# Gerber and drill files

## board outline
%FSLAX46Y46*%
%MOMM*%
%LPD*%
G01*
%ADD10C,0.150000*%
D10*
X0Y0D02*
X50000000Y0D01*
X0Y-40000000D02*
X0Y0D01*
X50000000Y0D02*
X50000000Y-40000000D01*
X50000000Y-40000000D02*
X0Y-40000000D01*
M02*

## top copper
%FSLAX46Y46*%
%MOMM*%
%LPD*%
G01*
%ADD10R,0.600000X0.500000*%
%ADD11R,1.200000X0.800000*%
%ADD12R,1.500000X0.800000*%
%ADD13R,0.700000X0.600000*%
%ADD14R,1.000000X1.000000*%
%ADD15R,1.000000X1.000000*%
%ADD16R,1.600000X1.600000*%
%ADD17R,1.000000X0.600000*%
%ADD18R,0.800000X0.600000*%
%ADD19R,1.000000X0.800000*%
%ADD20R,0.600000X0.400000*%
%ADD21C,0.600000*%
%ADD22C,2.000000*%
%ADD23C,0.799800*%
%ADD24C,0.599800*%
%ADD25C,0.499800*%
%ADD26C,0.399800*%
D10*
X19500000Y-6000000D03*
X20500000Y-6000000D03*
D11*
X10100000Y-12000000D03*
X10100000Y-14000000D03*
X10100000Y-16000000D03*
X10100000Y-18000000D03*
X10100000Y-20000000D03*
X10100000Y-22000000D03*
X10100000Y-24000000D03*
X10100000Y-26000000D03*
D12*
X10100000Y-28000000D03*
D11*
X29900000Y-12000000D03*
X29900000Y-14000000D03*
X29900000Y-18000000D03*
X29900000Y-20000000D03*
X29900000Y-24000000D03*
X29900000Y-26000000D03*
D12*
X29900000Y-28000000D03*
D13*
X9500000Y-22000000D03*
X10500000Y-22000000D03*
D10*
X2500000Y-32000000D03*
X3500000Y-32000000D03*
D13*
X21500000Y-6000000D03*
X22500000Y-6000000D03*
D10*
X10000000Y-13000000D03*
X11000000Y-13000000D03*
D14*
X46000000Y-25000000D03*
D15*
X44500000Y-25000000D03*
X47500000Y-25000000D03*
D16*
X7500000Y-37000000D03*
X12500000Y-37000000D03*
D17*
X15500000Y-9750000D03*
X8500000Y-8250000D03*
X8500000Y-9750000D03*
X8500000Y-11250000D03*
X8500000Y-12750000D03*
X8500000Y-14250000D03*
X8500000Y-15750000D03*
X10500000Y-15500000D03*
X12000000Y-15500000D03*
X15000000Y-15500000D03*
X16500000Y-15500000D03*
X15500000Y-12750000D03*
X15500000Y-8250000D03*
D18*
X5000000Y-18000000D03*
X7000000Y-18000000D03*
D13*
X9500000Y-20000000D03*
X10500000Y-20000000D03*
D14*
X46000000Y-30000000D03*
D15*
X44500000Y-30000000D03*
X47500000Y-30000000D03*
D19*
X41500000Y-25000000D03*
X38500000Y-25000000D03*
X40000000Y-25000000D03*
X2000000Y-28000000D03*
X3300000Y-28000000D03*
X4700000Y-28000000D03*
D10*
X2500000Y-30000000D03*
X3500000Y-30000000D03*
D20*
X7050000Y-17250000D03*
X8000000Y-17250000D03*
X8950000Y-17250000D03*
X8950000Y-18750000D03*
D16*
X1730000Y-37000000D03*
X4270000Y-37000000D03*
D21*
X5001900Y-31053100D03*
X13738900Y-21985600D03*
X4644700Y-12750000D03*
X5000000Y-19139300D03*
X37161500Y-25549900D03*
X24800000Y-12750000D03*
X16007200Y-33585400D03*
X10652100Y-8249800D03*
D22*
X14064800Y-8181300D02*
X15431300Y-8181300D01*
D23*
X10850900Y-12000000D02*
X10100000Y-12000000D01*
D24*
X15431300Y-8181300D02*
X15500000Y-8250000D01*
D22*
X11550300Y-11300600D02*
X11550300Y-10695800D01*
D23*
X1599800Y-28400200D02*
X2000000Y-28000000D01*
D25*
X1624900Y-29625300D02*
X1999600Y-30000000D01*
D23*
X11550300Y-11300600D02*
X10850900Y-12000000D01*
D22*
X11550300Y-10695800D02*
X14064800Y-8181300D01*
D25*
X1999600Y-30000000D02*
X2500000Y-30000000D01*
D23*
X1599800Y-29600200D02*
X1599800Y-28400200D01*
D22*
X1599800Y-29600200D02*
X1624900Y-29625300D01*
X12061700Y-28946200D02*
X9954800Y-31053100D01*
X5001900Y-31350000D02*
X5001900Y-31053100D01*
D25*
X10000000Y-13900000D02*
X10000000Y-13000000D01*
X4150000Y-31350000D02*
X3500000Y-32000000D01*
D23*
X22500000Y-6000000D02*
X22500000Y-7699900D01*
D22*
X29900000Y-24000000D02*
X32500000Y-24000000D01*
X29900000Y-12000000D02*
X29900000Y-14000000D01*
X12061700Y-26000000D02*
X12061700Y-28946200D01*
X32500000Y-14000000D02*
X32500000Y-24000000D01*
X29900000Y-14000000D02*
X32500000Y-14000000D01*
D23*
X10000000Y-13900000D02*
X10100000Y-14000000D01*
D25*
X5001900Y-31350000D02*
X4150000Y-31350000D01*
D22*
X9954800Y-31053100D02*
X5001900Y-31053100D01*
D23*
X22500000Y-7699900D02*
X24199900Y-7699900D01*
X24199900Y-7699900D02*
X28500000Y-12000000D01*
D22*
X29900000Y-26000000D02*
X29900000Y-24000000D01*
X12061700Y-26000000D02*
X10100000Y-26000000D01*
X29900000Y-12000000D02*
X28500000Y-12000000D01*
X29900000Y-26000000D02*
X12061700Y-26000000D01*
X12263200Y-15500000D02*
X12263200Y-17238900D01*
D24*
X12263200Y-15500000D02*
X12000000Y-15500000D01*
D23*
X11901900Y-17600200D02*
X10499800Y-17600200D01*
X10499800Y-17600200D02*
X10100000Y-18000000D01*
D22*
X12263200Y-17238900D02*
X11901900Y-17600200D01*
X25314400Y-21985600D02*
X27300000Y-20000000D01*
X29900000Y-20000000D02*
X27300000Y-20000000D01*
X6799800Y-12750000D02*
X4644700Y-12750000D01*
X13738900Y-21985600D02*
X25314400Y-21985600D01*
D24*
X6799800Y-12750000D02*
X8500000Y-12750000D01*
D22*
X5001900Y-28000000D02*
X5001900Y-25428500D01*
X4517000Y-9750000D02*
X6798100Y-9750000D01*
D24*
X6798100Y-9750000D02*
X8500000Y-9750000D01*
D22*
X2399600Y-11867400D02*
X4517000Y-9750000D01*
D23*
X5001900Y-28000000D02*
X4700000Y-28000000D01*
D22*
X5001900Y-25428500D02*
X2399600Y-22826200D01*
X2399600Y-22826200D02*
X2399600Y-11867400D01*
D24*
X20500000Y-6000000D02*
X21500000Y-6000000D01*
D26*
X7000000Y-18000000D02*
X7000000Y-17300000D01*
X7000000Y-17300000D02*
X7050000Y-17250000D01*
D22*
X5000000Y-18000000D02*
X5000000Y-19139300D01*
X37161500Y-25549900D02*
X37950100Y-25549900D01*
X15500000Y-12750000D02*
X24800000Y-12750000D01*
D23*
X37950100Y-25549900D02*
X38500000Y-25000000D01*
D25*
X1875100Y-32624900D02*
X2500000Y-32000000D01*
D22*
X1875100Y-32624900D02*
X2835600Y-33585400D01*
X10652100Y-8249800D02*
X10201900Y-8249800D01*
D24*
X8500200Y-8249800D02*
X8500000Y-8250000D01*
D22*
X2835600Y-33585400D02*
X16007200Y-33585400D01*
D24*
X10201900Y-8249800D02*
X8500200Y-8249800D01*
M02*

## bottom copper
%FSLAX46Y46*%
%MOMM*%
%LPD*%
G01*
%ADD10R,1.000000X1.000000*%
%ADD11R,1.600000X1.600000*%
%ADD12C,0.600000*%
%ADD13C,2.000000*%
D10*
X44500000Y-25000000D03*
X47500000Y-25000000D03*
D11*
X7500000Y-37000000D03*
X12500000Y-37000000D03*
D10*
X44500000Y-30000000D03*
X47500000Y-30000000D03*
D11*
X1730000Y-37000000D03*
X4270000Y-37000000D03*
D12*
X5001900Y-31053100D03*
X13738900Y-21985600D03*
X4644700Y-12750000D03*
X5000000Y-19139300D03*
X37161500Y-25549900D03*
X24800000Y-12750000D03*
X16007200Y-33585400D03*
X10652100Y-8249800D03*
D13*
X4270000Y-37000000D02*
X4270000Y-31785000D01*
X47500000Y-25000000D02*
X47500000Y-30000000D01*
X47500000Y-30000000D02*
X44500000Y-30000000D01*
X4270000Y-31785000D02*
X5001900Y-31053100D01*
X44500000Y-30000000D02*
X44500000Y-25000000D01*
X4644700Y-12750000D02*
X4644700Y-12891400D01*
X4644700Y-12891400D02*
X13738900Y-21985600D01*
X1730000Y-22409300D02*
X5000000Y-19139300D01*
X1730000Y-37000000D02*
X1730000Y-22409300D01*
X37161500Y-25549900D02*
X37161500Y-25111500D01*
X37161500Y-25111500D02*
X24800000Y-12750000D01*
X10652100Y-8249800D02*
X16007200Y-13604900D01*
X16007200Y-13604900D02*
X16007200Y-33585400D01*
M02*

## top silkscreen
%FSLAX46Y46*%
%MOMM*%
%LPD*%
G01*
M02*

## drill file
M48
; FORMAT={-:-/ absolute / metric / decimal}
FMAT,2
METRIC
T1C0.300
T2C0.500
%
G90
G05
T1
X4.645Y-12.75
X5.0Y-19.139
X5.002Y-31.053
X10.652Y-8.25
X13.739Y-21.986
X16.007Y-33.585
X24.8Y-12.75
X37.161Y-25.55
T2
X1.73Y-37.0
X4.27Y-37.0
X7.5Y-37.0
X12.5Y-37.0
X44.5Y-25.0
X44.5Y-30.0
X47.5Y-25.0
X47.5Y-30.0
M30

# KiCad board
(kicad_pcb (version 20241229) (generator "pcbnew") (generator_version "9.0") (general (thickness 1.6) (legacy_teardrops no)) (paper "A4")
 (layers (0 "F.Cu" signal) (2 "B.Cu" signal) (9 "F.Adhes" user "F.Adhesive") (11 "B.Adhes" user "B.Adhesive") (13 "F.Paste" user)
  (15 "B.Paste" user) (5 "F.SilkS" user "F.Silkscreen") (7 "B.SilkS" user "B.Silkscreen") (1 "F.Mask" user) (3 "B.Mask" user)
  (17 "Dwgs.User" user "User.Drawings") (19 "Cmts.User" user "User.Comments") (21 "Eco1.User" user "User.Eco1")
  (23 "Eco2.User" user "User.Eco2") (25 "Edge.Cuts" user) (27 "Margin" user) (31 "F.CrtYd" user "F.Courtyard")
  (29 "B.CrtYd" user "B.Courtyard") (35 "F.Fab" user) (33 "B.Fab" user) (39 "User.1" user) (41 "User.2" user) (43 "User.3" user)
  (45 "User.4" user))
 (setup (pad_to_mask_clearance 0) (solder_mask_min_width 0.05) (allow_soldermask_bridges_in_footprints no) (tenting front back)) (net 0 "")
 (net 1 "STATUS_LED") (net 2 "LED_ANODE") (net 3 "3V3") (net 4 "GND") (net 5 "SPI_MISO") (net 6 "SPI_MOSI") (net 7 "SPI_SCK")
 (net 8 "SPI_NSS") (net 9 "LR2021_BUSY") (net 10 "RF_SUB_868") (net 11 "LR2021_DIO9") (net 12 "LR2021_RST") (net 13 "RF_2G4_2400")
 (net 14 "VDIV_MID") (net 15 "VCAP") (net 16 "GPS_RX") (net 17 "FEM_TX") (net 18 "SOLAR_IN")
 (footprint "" (layer "F.Cu") (at 20 6)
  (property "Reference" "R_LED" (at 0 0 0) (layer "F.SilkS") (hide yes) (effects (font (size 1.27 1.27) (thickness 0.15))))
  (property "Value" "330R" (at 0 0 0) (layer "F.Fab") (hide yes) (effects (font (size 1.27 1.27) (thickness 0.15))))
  (pad "1" smd rect (at -0.5 0) (size 0.6 0.5) (layers "F.Cu" "F.Mask") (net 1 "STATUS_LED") (thermal_bridge_angle 45))
  (pad "2" smd rect (at 0.5 0) (size 0.6 0.5) (layers "F.Cu" "F.Mask") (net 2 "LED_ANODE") (thermal_bridge_angle 45)))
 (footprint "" (layer "F.Cu") (at 20 20)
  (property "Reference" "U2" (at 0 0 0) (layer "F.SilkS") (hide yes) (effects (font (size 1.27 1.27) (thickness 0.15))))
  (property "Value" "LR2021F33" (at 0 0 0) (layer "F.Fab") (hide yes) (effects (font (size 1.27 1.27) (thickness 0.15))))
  (pad "1" smd rect (at -9.9 -8) (size 1.2 0.8) (layers "F.Cu" "F.Mask") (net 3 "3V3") (thermal_bridge_angle 45))
  (pad "2" smd rect (at -9.9 -6) (size 1.2 0.8) (layers "F.Cu" "F.Mask") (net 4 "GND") (thermal_bridge_angle 45))
  (pad "3" smd rect (at -9.9 -4) (size 1.2 0.8) (layers "F.Cu" "F.Mask") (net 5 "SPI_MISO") (thermal_bridge_angle 45))
  (pad "4" smd rect (at -9.9 -2) (size 1.2 0.8) (layers "F.Cu" "F.Mask") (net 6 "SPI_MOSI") (thermal_bridge_angle 45))
  (pad "5" smd rect (at -9.9 0) (size 1.2 0.8) (layers "F.Cu" "F.Mask") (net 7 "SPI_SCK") (thermal_bridge_angle 45))
  (pad "6" smd rect (at -9.9 2) (size 1.2 0.8) (layers "F.Cu" "F.Mask") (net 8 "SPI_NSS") (thermal_bridge_angle 45))
  (pad "7" smd rect (at -9.9 4) (size 1.2 0.8) (layers "F.Cu" "F.Mask") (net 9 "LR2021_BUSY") (thermal_bridge_angle 45))
  (pad "8" smd rect (at -9.9 6) (size 1.2 0.8) (layers "F.Cu" "F.Mask") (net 4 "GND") (thermal_bridge_angle 45))
  (pad "9" smd rect (at -9.9 8) (size 1.5 0.8) (layers "F.Cu" "F.Mask") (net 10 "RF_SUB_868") (thermal_bridge_angle 45))
  (pad "10" smd rect (at 9.9 -8) (size 1.2 0.8) (layers "F.Cu" "F.Mask") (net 4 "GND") (thermal_bridge_angle 45))
  (pad "11" smd rect (at 9.9 -6) (size 1.2 0.8) (layers "F.Cu" "F.Mask") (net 4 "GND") (thermal_bridge_angle 45))
  (pad "13" smd rect (at 9.9 -2) (size 1.2 0.8) (layers "F.Cu" "F.Mask") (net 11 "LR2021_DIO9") (thermal_bridge_angle 45))
  (pad "14" smd rect (at 9.9 0) (size 1.2 0.8) (layers "F.Cu" "F.Mask") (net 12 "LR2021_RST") (thermal_bridge_angle 45))
  (pad "16" smd rect (at 9.9 4) (size 1.2 0.8) (layers "F.Cu" "F.Mask") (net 4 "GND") (thermal_bridge_angle 45))
  (pad "17" smd rect (at 9.9 6) (size 1.2 0.8) (layers "F.Cu" "F.Mask") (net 4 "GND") (thermal_bridge_angle 45))
  (pad "18" smd rect (at 9.9 8) (size 1.5 0.8) (layers "F.Cu" "F.Mask") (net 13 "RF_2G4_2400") (thermal_bridge_angle 45)))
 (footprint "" (layer "F.Cu") (at 10 22)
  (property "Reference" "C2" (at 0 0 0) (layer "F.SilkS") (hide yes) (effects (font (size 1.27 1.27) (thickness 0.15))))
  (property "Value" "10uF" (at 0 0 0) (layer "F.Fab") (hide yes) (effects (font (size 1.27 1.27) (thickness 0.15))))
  (pad "1" smd rect (at -0.5 0) (size 0.7 0.6) (layers "F.Cu" "F.Mask") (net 3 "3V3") (thermal_bridge_angle 45))
  (pad "2" smd rect (at 0.5 0) (size 0.7 0.6) (layers "F.Cu" "F.Mask") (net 4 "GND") (thermal_bridge_angle 45)))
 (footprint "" (layer "F.Cu") (at 3 32)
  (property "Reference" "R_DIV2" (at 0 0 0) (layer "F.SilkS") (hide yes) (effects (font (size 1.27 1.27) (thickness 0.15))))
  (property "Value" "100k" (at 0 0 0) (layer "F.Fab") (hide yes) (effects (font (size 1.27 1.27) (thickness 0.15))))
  (pad "1" smd rect (at -0.5 0) (size 0.6 0.5) (layers "F.Cu" "F.Mask") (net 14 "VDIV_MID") (thermal_bridge_angle 45))
  (pad "2" smd rect (at 0.5 0) (size 0.6 0.5) (layers "F.Cu" "F.Mask") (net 4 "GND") (thermal_bridge_angle 45)))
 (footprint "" (layer "F.Cu") (at 22 6)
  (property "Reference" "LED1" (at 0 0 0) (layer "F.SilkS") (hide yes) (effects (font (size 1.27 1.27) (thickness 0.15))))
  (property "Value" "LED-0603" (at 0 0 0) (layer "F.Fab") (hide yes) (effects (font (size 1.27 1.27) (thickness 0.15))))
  (pad "A" smd rect (at -0.5 0) (size 0.7 0.6) (layers "F.Cu" "F.Mask") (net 2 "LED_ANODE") (thermal_bridge_angle 45))
  (pad "K" smd rect (at 0.5 0) (size 0.7 0.6) (layers "F.Cu" "F.Mask") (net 4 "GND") (thermal_bridge_angle 45)))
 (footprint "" (layer "F.Cu") (at 10.5 13)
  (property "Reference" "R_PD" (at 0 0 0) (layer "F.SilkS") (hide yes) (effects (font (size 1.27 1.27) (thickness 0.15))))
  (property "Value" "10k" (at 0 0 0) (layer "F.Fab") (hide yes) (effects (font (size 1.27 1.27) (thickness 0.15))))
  (pad "1" smd rect (at -0.5 0) (size 0.6 0.5) (layers "F.Cu" "F.Mask") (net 4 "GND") (thermal_bridge_angle 45))
  (pad "2" smd rect (at 0.5 0) (size 0.6 0.5) (layers "F.Cu" "F.Mask") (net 5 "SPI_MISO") (thermal_bridge_angle 45)))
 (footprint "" (layer "F.Cu") (at 46 25)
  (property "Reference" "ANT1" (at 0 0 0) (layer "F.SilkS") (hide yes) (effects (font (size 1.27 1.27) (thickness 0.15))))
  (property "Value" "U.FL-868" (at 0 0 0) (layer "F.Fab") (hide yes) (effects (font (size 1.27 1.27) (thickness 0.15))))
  (pad "1" smd rect (at 0 0) (size 1 1) (layers "F.Cu" "F.Mask") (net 10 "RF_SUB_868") (thermal_bridge_angle 45))
  (pad "2" thru_hole rect (at -1.5 0) (size 1 1) (drill 0.5) (layers "*.Cu" "*.Mask") (remove_unused_layers no) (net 4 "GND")
   (thermal_bridge_angle 45))
  (pad "3" thru_hole rect (at 1.5 0) (size 1 1) (drill 0.5) (layers "*.Cu" "*.Mask") (remove_unused_layers no) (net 4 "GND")
   (thermal_bridge_angle 45)))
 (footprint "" (layer "F.Cu") (at 10 37)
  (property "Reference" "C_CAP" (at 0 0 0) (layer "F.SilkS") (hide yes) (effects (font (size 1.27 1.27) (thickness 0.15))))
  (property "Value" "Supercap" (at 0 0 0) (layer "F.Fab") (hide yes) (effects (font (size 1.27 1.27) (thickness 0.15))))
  (pad "1" thru_hole rect (at -2.5 0) (size 1.6 1.6) (drill 0.5) (layers "*.Cu" "*.Mask") (remove_unused_layers no) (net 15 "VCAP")
   (thermal_bridge_angle 45))
  (pad "2" thru_hole rect (at 2.5 0) (size 1.6 1.6) (drill 0.5) (layers "*.Cu" "*.Mask") (remove_unused_layers no) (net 4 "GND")
   (thermal_bridge_angle 45)))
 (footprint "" (layer "F.Cu") (at 12 12)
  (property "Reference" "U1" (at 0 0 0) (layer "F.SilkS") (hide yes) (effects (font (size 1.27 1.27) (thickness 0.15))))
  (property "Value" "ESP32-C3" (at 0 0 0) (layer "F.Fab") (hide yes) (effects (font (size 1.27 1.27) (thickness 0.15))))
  (pad "GND" smd rect (at 3.5 -2.25) (size 1 0.6) (layers "F.Cu" "F.Mask") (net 4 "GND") (thermal_bridge_angle 45))
  (pad "GPIO0" smd rect (at -3.5 -3.75) (size 1 0.6) (layers "F.Cu" "F.Mask") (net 14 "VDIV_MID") (thermal_bridge_angle 45))
  (pad "GPIO1" smd rect (at -3.5 -2.25) (size 1 0.6) (layers "F.Cu" "F.Mask") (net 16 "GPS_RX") (thermal_bridge_angle 45))
  (pad "GPIO2" smd rect (at -3.5 -0.75) (size 1 0.6) (layers "F.Cu" "F.Mask") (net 5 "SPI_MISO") (thermal_bridge_angle 45))
  (pad "GPIO3" smd rect (at -3.5 0.75) (size 1 0.6) (layers "F.Cu" "F.Mask") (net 12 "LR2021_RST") (thermal_bridge_angle 45))
  (pad "GPIO4" smd rect (at -3.5 2.25) (size 1 0.6) (layers "F.Cu" "F.Mask") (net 9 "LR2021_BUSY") (thermal_bridge_angle 45))
  (pad "GPIO5" smd rect (at -3.5 3.75) (size 1 0.6) (layers "F.Cu" "F.Mask") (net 11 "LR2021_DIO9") (thermal_bridge_angle 45))
  (pad "GPIO6" smd rect (at -1.5 3.5) (size 1 0.6) (layers "F.Cu" "F.Mask") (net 7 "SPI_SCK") (thermal_bridge_angle 45))
  (pad "GPIO7" smd rect (at 0 3.5) (size 1 0.6) (layers "F.Cu" "F.Mask") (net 6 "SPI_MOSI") (thermal_bridge_angle 45))
  (pad "GPIO9" smd rect (at 3 3.5) (size 1 0.6) (layers "F.Cu" "F.Mask") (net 1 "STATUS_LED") (thermal_bridge_angle 45))
  (pad "GPIO10" smd rect (at 4.5 3.5) (size 1 0.6) (layers "F.Cu" "F.Mask") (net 8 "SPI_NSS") (thermal_bridge_angle 45))
  (pad "GPIO19" smd rect (at 3.5 0.75) (size 1 0.6) (layers "F.Cu" "F.Mask") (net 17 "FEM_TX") (thermal_bridge_angle 45))
  (pad "VCC" smd rect (at 3.5 -3.75) (size 1 0.6) (layers "F.Cu" "F.Mask") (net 3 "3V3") (thermal_bridge_angle 45)))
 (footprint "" (layer "F.Cu") (at 6 18)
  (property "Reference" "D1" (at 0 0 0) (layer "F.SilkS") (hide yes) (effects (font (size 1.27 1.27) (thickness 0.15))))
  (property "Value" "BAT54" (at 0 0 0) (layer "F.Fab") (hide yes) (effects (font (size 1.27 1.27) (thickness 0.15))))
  (pad "A" smd rect (at -1 0) (size 0.8 0.6) (layers "F.Cu" "F.Mask") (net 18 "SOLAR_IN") (thermal_bridge_angle 45))
  (pad "K" smd rect (at 1 0) (size 0.8 0.6) (layers "F.Cu" "F.Mask") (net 15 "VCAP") (thermal_bridge_angle 45)))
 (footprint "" (layer "F.Cu") (at 10 20)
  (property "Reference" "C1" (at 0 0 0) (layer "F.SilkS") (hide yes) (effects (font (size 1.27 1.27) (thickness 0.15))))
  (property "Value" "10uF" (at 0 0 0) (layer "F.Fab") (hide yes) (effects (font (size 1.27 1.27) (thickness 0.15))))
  (pad "1" smd rect (at -0.5 0) (size 0.7 0.6) (layers "F.Cu" "F.Mask") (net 15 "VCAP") (thermal_bridge_angle 45))
  (pad "2" smd rect (at 0.5 0) (size 0.7 0.6) (layers "F.Cu" "F.Mask") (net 4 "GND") (thermal_bridge_angle 45)))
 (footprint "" (layer "F.Cu") (at 46 30)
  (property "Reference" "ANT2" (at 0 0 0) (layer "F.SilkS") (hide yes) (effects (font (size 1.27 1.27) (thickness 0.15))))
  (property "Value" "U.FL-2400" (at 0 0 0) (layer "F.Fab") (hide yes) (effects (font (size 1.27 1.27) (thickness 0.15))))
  (pad "1" smd rect (at 0 0) (size 1 1) (layers "F.Cu" "F.Mask") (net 13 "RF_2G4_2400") (thermal_bridge_angle 45))
  (pad "2" thru_hole rect (at -1.5 0) (size 1 1) (drill 0.5) (layers "*.Cu" "*.Mask") (remove_unused_layers no) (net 4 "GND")
   (thermal_bridge_angle 45))
  (pad "3" thru_hole rect (at 1.5 0) (size 1 1) (drill 0.5) (layers "*.Cu" "*.Mask") (remove_unused_layers no) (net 4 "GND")
   (thermal_bridge_angle 45)))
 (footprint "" (layer "F.Cu") (at 40 25)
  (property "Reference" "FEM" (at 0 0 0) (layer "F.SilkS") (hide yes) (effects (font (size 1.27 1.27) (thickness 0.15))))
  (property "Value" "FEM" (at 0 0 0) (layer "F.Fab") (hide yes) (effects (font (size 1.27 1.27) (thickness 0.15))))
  (pad "GND" smd rect (at 1.5 0) (size 1 0.8) (layers "F.Cu" "F.Mask") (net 4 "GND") (thermal_bridge_angle 45))
  (pad "TX" smd rect (at -1.5 0) (size 1 0.8) (layers "F.Cu" "F.Mask") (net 17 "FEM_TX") (thermal_bridge_angle 45))
  (pad "VCC" smd rect (at 0 0) (size 1 0.8) (layers "F.Cu" "F.Mask") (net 3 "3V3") (thermal_bridge_angle 45)))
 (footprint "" (layer "F.Cu") (at 4 28)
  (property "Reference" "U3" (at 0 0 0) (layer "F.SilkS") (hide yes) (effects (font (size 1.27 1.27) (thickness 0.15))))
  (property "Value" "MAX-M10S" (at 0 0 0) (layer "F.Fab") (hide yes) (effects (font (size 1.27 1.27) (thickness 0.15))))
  (pad "1" smd rect (at -2 0) (size 1 0.8) (layers "F.Cu" "F.Mask") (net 3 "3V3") (thermal_bridge_angle 45))
  (pad "2" smd rect (at -0.7 0) (size 1 0.8) (layers "F.Cu" "F.Mask") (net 4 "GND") (thermal_bridge_angle 45))
  (pad "3" smd rect (at 0.7 0) (size 1 0.8) (layers "F.Cu" "F.Mask") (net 16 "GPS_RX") (thermal_bridge_angle 45)))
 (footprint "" (layer "F.Cu") (at 3 30)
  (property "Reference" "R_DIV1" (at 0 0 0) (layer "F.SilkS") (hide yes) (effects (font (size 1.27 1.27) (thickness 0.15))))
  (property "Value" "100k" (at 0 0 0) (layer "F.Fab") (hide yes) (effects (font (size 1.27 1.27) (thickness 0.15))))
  (pad "1" smd rect (at -0.5 0) (size 0.6 0.5) (layers "F.Cu" "F.Mask") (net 3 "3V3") (thermal_bridge_angle 45))
  (pad "2" smd rect (at 0.5 0) (size 0.6 0.5) (layers "F.Cu" "F.Mask") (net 14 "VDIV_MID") (thermal_bridge_angle 45)))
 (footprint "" (layer "F.Cu") (at 8 18)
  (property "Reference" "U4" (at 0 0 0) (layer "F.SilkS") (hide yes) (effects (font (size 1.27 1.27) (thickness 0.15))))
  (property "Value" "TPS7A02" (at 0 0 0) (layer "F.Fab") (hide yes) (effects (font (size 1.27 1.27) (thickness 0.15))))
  (pad "1" smd rect (at -0.95 -0.75) (size 0.6 0.4) (layers "F.Cu" "F.Mask") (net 15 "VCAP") (thermal_bridge_angle 45))
  (pad "2" smd rect (at 0 -0.75) (size 0.6 0.4) (layers "F.Cu" "F.Mask") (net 4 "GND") (thermal_bridge_angle 45))
  (pad "3" smd rect (at 0.95 -0.75) (size 0.6 0.4) (layers "F.Cu" "F.Mask") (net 15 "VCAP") (thermal_bridge_angle 45))
  (pad "4" smd rect (at 0.95 0.75) (size 0.6 0.4) (layers "F.Cu" "F.Mask") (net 3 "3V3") (thermal_bridge_angle 45)))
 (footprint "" (layer "F.Cu") (at 3 37)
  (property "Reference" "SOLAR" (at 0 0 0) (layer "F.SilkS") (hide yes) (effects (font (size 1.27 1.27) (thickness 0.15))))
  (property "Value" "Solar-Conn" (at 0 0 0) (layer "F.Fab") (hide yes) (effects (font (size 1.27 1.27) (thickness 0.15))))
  (pad "1" thru_hole rect (at -1.27 0) (size 1.6 1.6) (drill 0.5) (layers "*.Cu" "*.Mask") (remove_unused_layers no) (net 18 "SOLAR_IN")
   (thermal_bridge_angle 45))
  (pad "2" thru_hole rect (at 1.27 0) (size 1.6 1.6) (drill 0.5) (layers "*.Cu" "*.Mask") (remove_unused_layers no) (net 4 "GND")
   (thermal_bridge_angle 45)))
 (gr_line (start 0 0) (end 50 0) (stroke (width 0.15) (type default)) (layer "Edge.Cuts"))
 (gr_line (start 0 40) (end 0 0) (stroke (width 0.15) (type default)) (layer "Edge.Cuts"))
 (gr_line (start 50 0) (end 50 40) (stroke (width 0.15) (type default)) (layer "Edge.Cuts"))
 (gr_line (start 50 40) (end 0 40) (stroke (width 0.15) (type default)) (layer "Edge.Cuts"))
 (segment (start 14.0648 8.1813) (end 15.4313 8.1813) (width 2) (layer "F.Cu") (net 3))
 (segment (start 10.8509 12) (end 10.1 12) (width 0.7998) (layer "F.Cu") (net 3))
 (segment (start 15.4313 8.1813) (end 15.5 8.25) (width 0.5998) (layer "F.Cu") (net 3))
 (segment (start 11.5503 11.3006) (end 11.5503 10.6958) (width 2) (layer "F.Cu") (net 3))
 (segment (start 1.5998 28.4002) (end 2 28) (width 0.7998) (layer "F.Cu") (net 3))
 (segment (start 1.6249 29.6253) (end 1.9996 30) (width 0.4998) (layer "F.Cu") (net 3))
 (segment (start 11.5503 11.3006) (end 10.8509 12) (width 0.7998) (layer "F.Cu") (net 3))
 (segment (start 11.5503 10.6958) (end 14.0648 8.1813) (width 2) (layer "F.Cu") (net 3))
 (segment (start 1.9996 30) (end 2.5 30) (width 0.4998) (layer "F.Cu") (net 3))
 (segment (start 1.5998 29.6002) (end 1.5998 28.4002) (width 0.7998) (layer "F.Cu") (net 3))
 (segment (start 1.5998 29.6002) (end 1.6249 29.6253) (width 2) (layer "F.Cu") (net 3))
 (segment (start 12.0617 28.9462) (end 9.9548 31.0531) (width 2) (layer "F.Cu") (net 4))
 (segment (start 5.0019 31.35) (end 5.0019 31.0531) (width 2) (layer "F.Cu") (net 4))
 (segment (start 10 13.9) (end 10 13) (width 0.4998) (layer "F.Cu") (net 4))
 (segment (start 4.15 31.35) (end 3.5 32) (width 0.4998) (layer "F.Cu") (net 4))
 (segment (start 22.5 6) (end 22.5 7.6999) (width 0.7998) (layer "F.Cu") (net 4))
 (segment (start 29.9 24) (end 32.5 24) (width 2) (layer "F.Cu") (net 4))
 (segment (start 29.9 12) (end 29.9 14) (width 2) (layer "F.Cu") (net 4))
 (segment (start 12.0617 26) (end 12.0617 28.9462) (width 2) (layer "F.Cu") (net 4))
 (segment (start 32.5 14) (end 32.5 24) (width 2) (layer "F.Cu") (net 4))
 (segment (start 29.9 14) (end 32.5 14) (width 2) (layer "F.Cu") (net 4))
 (segment (start 10 13.9) (end 10.1 14) (width 0.7998) (layer "F.Cu") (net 4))
 (segment (start 5.0019 31.35) (end 4.15 31.35) (width 0.4998) (layer "F.Cu") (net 4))
 (segment (start 9.9548 31.0531) (end 5.0019 31.0531) (width 2) (layer "F.Cu") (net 4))
 (segment (start 22.5 7.6999) (end 24.1999 7.6999) (width 0.7998) (layer "F.Cu") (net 4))
 (segment (start 24.1999 7.6999) (end 28.5 12) (width 0.7998) (layer "F.Cu") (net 4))
 (segment (start 29.9 26) (end 29.9 24) (width 2) (layer "F.Cu") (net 4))
 (segment (start 12.0617 26) (end 10.1 26) (width 2) (layer "F.Cu") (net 4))
 (segment (start 29.9 12) (end 28.5 12) (width 2) (layer "F.Cu") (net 4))
 (segment (start 29.9 26) (end 12.0617 26) (width 2) (layer "F.Cu") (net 4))
 (via (at 5.0019 31.0531) (size 0.6) (drill 0.3) (layers "F.Cu" "B.Cu") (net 4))
 (segment (start 4.27 37) (end 4.27 31.785) (width 2) (layer "B.Cu") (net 4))
 (segment (start 47.5 25) (end 47.5 30) (width 2) (layer "B.Cu") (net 4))
 (segment (start 47.5 30) (end 44.5 30) (width 2) (layer "B.Cu") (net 4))
 (segment (start 4.27 31.785) (end 5.0019 31.0531) (width 2) (layer "B.Cu") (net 4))
 (segment (start 44.5 30) (end 44.5 25) (width 2) (layer "B.Cu") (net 4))
 (segment (start 12.2632 15.5) (end 12.2632 17.2389) (width 2) (layer "F.Cu") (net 6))
 (segment (start 12.2632 15.5) (end 12 15.5) (width 0.5998) (layer "F.Cu") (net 6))
 (segment (start 11.9019 17.6002) (end 10.4998 17.6002) (width 0.7998) (layer "F.Cu") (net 6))
 (segment (start 10.4998 17.6002) (end 10.1 18) (width 0.7998) (layer "F.Cu") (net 6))
 (segment (start 12.2632 17.2389) (end 11.9019 17.6002) (width 2) (layer "F.Cu") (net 6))
 (segment (start 25.3144 21.9856) (end 27.3 20) (width 2) (layer "F.Cu") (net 12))
 (segment (start 29.9 20) (end 27.3 20) (width 2) (layer "F.Cu") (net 12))
 (segment (start 6.7998 12.75) (end 4.6447 12.75) (width 2) (layer "F.Cu") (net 12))
 (segment (start 13.7389 21.9856) (end 25.3144 21.9856) (width 2) (layer "F.Cu") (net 12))
 (segment (start 6.7998 12.75) (end 8.5 12.75) (width 0.5998) (layer "F.Cu") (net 12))
 (via (at 13.7389 21.9856) (size 0.6) (drill 0.3) (layers "F.Cu" "B.Cu") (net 12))
 (via (at 4.6447 12.75) (size 0.6) (drill 0.3) (layers "F.Cu" "B.Cu") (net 12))
 (segment (start 4.6447 12.75) (end 4.6447 12.8914) (width 2) (layer "B.Cu") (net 12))
 (segment (start 4.6447 12.8914) (end 13.7389 21.9856) (width 2) (layer "B.Cu") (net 12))
 (segment (start 5.0019 28) (end 5.0019 25.4285) (width 2) (layer "F.Cu") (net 16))
 (segment (start 4.517 9.75) (end 6.7981 9.75) (width 2) (layer "F.Cu") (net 16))
 (segment (start 6.7981 9.75) (end 8.5 9.75) (width 0.5998) (layer "F.Cu") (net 16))
 (segment (start 2.3996 11.8674) (end 4.517 9.75) (width 2) (layer "F.Cu") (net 16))
 (segment (start 5.0019 28) (end 4.7 28) (width 0.7998) (layer "F.Cu") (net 16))
 (segment (start 5.0019 25.4285) (end 2.3996 22.8262) (width 2) (layer "F.Cu") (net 16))
 (segment (start 2.3996 22.8262) (end 2.3996 11.8674) (width 2) (layer "F.Cu") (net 16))
 (segment (start 20.5 6) (end 21.5 6) (width 0.5998) (layer "F.Cu") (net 2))
 (segment (start 7 18) (end 7 17.3) (width 0.3998) (layer "F.Cu") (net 15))
 (segment (start 7 17.3) (end 7.05 17.25) (width 0.3998) (layer "F.Cu") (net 15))
 (segment (start 5 18) (end 5 19.1393) (width 2) (layer "F.Cu") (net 18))
 (via (at 5 19.1393) (size 0.6) (drill 0.3) (layers "F.Cu" "B.Cu") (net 18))
 (segment (start 1.73 22.4093) (end 5 19.1393) (width 2) (layer "B.Cu") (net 18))
 (segment (start 1.73 37) (end 1.73 22.4093) (width 2) (layer "B.Cu") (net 18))
 (segment (start 37.1615 25.5499) (end 37.9501 25.5499) (width 2) (layer "F.Cu") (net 17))
 (segment (start 15.5 12.75) (end 24.8 12.75) (width 2) (layer "F.Cu") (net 17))
 (segment (start 37.9501 25.5499) (end 38.5 25) (width 0.7998) (layer "F.Cu") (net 17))
 (via (at 37.1615 25.5499) (size 0.6) (drill 0.3) (layers "F.Cu" "B.Cu") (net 17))
 (via (at 24.8 12.75) (size 0.6) (drill 0.3) (layers "F.Cu" "B.Cu") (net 17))
 (segment (start 37.1615 25.5499) (end 37.1615 25.1115) (width 2) (layer "B.Cu") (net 17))
 (segment (start 37.1615 25.1115) (end 24.8 12.75) (width 2) (layer "B.Cu") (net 17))
 (segment (start 1.8751 32.6249) (end 2.5 32) (width 0.4998) (layer "F.Cu") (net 14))
 (segment (start 1.8751 32.6249) (end 2.8356 33.5854) (width 2) (layer "F.Cu") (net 14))
 (segment (start 10.6521 8.2498) (end 10.2019 8.2498) (width 2) (layer "F.Cu") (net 14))
 (segment (start 8.5002 8.2498) (end 8.5 8.25) (width 0.5998) (layer "F.Cu") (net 14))
 (segment (start 2.8356 33.5854) (end 16.0072 33.5854) (width 2) (layer "F.Cu") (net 14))
 (segment (start 10.2019 8.2498) (end 8.5002 8.2498) (width 0.5998) (layer "F.Cu") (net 14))
 (via (at 16.0072 33.5854) (size 0.6) (drill 0.3) (layers "F.Cu" "B.Cu") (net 14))
 (via (at 10.6521 8.2498) (size 0.6) (drill 0.3) (layers "F.Cu" "B.Cu") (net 14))
 (segment (start 10.6521 8.2498) (end 16.0072 13.6049) (width 2) (layer "B.Cu") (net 14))
 (segment (start 16.0072 13.6049) (end 16.0072 33.5854) (width 2) (layer "B.Cu") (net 14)))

